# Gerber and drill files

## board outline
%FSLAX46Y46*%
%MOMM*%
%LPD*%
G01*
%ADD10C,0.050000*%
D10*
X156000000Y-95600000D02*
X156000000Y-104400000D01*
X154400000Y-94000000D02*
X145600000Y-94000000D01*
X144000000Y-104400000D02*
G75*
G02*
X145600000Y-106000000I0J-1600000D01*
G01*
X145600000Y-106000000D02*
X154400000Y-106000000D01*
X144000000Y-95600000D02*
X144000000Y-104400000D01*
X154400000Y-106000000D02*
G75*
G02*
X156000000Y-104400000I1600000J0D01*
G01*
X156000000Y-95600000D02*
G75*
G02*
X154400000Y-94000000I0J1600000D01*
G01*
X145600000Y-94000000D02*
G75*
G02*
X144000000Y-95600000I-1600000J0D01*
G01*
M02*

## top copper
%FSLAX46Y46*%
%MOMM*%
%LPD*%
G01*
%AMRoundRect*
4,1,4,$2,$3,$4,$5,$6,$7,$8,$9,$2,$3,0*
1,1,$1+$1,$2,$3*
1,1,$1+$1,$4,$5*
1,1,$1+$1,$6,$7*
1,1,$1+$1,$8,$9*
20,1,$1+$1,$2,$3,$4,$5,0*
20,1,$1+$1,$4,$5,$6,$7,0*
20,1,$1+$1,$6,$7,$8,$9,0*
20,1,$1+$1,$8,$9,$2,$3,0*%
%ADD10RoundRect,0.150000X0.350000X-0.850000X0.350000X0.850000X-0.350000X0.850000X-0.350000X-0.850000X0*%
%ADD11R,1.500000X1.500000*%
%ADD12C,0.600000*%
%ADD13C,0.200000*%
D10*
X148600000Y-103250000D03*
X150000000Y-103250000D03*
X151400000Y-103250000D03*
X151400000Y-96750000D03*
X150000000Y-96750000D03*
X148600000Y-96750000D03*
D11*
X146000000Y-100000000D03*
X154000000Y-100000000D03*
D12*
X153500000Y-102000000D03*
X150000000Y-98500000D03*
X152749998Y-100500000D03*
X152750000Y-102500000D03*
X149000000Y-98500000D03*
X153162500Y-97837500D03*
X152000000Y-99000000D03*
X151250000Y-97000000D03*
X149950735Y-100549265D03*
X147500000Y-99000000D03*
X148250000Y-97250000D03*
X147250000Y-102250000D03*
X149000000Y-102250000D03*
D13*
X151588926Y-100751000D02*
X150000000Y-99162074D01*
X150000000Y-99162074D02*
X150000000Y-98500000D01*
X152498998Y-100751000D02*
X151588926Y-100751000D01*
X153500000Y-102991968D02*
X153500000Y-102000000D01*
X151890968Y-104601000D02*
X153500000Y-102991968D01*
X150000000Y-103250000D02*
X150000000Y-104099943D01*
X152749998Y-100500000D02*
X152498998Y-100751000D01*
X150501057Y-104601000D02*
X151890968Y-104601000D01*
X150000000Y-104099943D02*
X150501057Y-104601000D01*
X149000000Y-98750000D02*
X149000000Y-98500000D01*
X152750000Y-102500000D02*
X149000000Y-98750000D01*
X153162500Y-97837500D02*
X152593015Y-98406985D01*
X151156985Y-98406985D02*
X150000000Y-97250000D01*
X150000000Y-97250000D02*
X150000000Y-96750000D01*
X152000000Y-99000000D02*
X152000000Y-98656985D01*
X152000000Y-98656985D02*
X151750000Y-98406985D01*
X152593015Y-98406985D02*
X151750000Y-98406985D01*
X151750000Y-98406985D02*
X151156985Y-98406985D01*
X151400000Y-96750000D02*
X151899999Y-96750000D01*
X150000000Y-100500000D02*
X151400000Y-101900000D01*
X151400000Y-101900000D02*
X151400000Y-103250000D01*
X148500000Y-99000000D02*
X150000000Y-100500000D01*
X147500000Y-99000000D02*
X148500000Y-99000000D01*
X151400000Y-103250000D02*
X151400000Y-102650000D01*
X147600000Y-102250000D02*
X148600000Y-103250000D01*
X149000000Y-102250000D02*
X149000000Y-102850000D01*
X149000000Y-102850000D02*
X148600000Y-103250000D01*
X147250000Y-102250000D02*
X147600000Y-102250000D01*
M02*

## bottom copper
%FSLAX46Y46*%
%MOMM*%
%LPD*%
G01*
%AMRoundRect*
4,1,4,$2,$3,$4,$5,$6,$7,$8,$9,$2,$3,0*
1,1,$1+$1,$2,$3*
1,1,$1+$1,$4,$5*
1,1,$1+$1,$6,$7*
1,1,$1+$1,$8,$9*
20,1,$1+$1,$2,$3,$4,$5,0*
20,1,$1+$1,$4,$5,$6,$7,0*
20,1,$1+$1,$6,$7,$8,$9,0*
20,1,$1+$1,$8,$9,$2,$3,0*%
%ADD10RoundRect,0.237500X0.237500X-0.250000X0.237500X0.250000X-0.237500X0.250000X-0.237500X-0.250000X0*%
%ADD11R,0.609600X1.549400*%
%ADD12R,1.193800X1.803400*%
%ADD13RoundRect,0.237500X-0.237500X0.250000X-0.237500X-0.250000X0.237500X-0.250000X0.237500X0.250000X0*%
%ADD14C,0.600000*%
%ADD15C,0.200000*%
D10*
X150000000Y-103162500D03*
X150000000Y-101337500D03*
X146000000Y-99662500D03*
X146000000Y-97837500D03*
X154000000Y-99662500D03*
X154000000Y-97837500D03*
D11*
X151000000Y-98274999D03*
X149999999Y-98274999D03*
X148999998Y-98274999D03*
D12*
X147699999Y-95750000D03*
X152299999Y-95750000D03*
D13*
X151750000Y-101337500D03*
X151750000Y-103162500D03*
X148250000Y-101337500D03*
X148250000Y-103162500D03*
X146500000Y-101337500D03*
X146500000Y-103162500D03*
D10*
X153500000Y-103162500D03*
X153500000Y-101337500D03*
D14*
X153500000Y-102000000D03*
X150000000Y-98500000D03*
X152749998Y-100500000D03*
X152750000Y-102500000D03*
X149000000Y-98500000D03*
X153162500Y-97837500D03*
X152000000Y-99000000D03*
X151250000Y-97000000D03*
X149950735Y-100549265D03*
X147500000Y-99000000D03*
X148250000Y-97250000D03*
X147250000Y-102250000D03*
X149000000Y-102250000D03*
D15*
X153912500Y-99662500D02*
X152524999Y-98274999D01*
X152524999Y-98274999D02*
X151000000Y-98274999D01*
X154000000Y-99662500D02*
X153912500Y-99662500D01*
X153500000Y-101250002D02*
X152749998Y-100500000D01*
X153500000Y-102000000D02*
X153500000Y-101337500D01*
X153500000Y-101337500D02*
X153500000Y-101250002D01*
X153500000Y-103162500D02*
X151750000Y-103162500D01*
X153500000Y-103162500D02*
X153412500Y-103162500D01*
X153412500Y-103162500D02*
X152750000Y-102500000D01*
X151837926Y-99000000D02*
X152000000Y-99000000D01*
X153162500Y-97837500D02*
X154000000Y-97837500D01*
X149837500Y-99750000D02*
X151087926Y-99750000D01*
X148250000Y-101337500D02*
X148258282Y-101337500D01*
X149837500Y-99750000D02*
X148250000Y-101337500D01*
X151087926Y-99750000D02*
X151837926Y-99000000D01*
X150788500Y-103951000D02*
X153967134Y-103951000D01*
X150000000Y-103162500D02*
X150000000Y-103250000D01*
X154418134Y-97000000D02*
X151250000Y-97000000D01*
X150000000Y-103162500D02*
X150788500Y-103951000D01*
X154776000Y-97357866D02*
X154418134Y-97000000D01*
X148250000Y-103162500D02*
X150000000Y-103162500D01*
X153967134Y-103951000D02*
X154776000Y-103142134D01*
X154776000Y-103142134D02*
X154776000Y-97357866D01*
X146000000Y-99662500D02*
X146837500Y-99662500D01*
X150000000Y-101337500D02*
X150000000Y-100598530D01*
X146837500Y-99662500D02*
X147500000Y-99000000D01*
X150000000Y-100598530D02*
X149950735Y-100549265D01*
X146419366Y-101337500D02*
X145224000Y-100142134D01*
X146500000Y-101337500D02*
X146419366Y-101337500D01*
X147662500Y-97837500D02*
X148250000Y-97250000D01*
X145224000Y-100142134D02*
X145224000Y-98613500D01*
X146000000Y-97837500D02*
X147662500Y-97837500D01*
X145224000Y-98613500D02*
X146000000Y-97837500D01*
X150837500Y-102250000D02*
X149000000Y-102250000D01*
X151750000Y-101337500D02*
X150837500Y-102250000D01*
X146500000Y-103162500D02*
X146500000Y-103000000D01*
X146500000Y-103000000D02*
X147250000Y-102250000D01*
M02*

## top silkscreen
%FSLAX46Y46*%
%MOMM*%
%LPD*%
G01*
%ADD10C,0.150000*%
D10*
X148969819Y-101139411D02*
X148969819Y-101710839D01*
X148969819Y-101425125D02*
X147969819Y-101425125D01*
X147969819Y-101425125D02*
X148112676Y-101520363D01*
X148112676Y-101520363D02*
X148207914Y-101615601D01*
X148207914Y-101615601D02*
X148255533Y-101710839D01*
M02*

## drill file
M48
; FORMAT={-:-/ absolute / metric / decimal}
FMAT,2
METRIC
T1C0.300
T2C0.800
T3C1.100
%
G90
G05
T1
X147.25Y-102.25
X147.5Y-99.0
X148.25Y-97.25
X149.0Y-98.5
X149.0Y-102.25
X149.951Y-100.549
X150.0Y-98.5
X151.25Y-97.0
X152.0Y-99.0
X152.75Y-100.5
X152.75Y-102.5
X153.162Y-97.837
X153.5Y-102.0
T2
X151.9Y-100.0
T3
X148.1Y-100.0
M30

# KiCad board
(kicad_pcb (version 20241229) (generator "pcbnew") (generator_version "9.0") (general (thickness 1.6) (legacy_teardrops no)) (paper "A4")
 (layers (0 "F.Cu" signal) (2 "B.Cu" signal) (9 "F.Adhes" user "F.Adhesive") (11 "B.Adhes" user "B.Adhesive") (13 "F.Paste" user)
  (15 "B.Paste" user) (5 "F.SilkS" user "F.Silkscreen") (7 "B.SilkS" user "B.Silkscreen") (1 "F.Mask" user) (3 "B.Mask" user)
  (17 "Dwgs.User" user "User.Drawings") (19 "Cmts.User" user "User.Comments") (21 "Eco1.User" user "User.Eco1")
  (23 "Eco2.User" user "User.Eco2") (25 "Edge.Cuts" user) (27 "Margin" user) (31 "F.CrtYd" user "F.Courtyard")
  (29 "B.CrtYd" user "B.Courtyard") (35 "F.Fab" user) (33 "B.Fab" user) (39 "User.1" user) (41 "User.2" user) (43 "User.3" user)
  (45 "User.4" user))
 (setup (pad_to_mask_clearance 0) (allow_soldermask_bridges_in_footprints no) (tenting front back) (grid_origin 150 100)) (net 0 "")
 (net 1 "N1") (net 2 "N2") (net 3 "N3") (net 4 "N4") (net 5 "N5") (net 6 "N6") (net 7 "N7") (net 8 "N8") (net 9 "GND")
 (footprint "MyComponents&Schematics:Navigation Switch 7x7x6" (layer "F.Cu") (at 150 100 90)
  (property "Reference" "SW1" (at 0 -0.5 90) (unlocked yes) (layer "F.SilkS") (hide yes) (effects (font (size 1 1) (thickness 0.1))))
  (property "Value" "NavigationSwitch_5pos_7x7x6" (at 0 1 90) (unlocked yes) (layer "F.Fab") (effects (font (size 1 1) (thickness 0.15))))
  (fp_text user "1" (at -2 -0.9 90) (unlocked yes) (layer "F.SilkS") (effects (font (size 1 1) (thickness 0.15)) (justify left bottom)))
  (pad "" np_thru_hole circle (at 0 -1.9 90) (size 1.1 1.1) (drill 1.1) (layers "*.Mask"))
  (pad "" np_thru_hole circle (at 0 1.9 90) (size 0.8 0.8) (drill 0.8) (layers "*.Mask"))
  (pad "1" smd roundrect (at -3.25 -1.4 90) (size 2 1) (layers "F.Cu" "F.Mask" "F.Paste") (roundrect_rratio 0.15) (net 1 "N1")
   (thermal_bridge_angle 45))
  (pad "2" smd roundrect (at -3.25 0 90) (size 2 1) (layers "F.Cu" "F.Mask" "F.Paste") (roundrect_rratio 0.15) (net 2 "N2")
   (thermal_bridge_angle 45))
  (pad "3" smd roundrect (at -3.25 1.4 90) (size 2 1) (layers "F.Cu" "F.Mask" "F.Paste") (roundrect_rratio 0.15) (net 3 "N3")
   (thermal_bridge_angle 45))
  (pad "4" smd roundrect (at 3.25 1.4 90) (size 2 1) (layers "F.Cu" "F.Mask" "F.Paste") (roundrect_rratio 0.15) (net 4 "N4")
   (thermal_bridge_angle 45))
  (pad "5" smd roundrect (at 3.25 0 90) (size 2 1) (layers "F.Cu" "F.Mask" "F.Paste") (roundrect_rratio 0.15) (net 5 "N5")
   (thermal_bridge_angle 45))
  (pad "6" smd roundrect (at 3.25 -1.4 90) (size 2 1) (layers "F.Cu" "F.Mask" "F.Paste") (roundrect_rratio 0.15) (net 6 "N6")
   (thermal_bridge_angle 45))
  (pad "MP" smd rect (at 0 -4 90) (size 1.5 1.5) (layers "F.Cu" "F.Mask" "F.Paste") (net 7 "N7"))
  (pad "MP" smd rect (at 0 4 90) (size 1.5 1.5) (layers "F.Cu" "F.Mask" "F.Paste") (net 7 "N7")))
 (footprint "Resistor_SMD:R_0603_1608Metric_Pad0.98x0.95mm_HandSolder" (layer "B.Cu") (at 150 102.25 90)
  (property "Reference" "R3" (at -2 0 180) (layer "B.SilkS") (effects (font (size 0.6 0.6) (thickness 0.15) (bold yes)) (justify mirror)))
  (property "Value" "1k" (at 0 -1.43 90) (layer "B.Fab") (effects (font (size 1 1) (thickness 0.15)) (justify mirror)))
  (pad "1" smd roundrect (at -0.9125 0 90) (size 0.975 0.95) (layers "B.Cu" "B.Mask" "B.Paste") (roundrect_rratio 0.25) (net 4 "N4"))
  (pad "2" smd roundrect (at 0.9125 0 90) (size 0.975 0.95) (layers "B.Cu" "B.Mask" "B.Paste") (roundrect_rratio 0.25) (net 3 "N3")))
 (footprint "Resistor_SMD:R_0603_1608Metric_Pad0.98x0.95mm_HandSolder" (layer "B.Cu") (at 146 98.75 90)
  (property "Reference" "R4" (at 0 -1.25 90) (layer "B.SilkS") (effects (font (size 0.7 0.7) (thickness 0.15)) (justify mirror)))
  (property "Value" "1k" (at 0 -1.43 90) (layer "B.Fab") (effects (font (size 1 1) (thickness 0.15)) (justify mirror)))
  (pad "1" smd roundrect (at -0.9125 0 90) (size 0.975 0.95) (layers "B.Cu" "B.Mask" "B.Paste") (roundrect_rratio 0.25) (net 3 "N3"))
  (pad "2" smd roundrect (at 0.9125 0 90) (size 0.975 0.95) (layers "B.Cu" "B.Mask" "B.Paste") (roundrect_rratio 0.25) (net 6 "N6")))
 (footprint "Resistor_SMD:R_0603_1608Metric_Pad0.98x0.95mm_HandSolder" (layer "B.Cu") (at 154 98.75 90)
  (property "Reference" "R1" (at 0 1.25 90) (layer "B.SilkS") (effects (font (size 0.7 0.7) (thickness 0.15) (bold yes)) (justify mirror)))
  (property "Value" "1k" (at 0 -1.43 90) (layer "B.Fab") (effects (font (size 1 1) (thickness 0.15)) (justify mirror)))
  (pad "1" smd roundrect (at -0.9125 0 90) (size 0.975 0.95) (layers "B.Cu" "B.Mask" "B.Paste") (roundrect_rratio 0.25) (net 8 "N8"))
  (pad "2" smd roundrect (at 0.9125 0 90) (size 0.975 0.95) (layers "B.Cu" "B.Mask" "B.Paste") (roundrect_rratio 0.25) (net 5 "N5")))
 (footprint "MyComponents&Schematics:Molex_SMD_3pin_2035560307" (layer "B.Cu") (at 149.999999 96.551399)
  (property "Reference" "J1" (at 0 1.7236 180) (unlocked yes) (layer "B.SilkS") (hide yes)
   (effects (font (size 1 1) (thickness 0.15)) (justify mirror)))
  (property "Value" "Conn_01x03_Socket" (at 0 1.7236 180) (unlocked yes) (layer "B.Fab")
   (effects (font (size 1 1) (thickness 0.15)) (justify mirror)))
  (pad "1" smd rect (at 1.000001 1.7236) (size 0.6096 1.5494) (layers "B.Cu" "B.Mask" "B.Paste") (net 8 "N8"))
  (pad "2" smd rect (at 0 1.7236) (size 0.6096 1.5494) (layers "B.Cu" "B.Mask" "B.Paste") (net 2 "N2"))
  (pad "3" smd rect (at -1.000001 1.7236) (size 0.6096 1.5494) (layers "B.Cu" "B.Mask" "B.Paste") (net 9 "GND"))
  (pad "4" smd rect (at -2.3 -0.801399) (size 1.1938 1.8034) (layers "B.Cu" "B.Mask" "B.Paste"))
  (pad "5" smd rect (at 2.3 -0.801399) (size 1.1938 1.8034) (layers "B.Cu" "B.Mask" "B.Paste")))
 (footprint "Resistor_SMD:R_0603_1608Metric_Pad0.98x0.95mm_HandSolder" (layer "B.Cu") (at 151.75 102.25 -90)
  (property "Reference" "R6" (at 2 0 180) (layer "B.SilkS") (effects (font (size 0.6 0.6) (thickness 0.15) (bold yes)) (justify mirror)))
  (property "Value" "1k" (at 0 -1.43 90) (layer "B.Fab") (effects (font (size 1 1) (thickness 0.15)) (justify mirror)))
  (pad "1" smd roundrect (at -0.9125 0 270) (size 0.975 0.95) (layers "B.Cu" "B.Mask" "B.Paste") (roundrect_rratio 0.25) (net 1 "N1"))
  (pad "2" smd roundrect (at 0.9125 0 270) (size 0.975 0.95) (layers "B.Cu" "B.Mask" "B.Paste") (roundrect_rratio 0.25) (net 9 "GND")))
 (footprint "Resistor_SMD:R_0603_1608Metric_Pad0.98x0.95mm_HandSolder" (layer "B.Cu") (at 148.25 102.25 -90)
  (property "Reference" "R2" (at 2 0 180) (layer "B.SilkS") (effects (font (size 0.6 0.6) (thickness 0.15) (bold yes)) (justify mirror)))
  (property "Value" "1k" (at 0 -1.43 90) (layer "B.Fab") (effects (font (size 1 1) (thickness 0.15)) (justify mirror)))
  (pad "1" smd roundrect (at -0.9125 0 270) (size 0.975 0.95) (layers "B.Cu" "B.Mask" "B.Paste") (roundrect_rratio 0.25) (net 5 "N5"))
  (pad "2" smd roundrect (at 0.9125 0 270) (size 0.975 0.95) (layers "B.Cu" "B.Mask" "B.Paste") (roundrect_rratio 0.25) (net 4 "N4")))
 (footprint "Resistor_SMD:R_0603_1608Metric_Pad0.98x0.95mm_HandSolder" (layer "B.Cu") (at 146.5 102.25 -90)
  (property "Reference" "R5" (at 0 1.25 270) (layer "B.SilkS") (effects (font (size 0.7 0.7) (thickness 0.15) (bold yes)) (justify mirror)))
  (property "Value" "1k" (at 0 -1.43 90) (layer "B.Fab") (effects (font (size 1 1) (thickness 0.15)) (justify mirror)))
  (pad "1" smd roundrect (at -0.9125 0 270) (size 0.975 0.95) (layers "B.Cu" "B.Mask" "B.Paste") (roundrect_rratio 0.25) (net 6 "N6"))
  (pad "2" smd roundrect (at 0.9125 0 270) (size 0.975 0.95) (layers "B.Cu" "B.Mask" "B.Paste") (roundrect_rratio 0.25) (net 1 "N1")))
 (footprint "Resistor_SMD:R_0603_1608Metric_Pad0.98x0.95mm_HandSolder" (layer "B.Cu") (at 153.5 102.25 90)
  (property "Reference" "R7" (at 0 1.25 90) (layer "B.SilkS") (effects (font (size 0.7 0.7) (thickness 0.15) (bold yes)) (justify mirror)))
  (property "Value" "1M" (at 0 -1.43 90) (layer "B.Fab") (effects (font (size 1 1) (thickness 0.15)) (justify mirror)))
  (pad "1" smd roundrect (at -0.9125 0 90) (size 0.975 0.95) (layers "B.Cu" "B.Mask" "B.Paste") (roundrect_rratio 0.25) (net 9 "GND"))
  (pad "2" smd roundrect (at 0.9125 0 90) (size 0.975 0.95) (layers "B.Cu" "B.Mask" "B.Paste") (roundrect_rratio 0.25) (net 2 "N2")))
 (gr_line (start 156 95.6) (end 156 104.4) (stroke (width 0.05) (type default)) (layer "Edge.Cuts"))
 (gr_line (start 154.4 94) (end 145.6 94) (stroke (width 0.05) (type default)) (layer "Edge.Cuts"))
 (gr_arc (start 144 104.4) (mid 145.131371 104.868629) (end 145.6 106) (stroke (width 0.05) (type default)) (layer "Edge.Cuts"))
 (gr_line (start 145.6 106) (end 154.4 106) (stroke (width 0.05) (type default)) (layer "Edge.Cuts"))
 (gr_line (start 144 95.6) (end 144 104.4) (stroke (width 0.05) (type default)) (layer "Edge.Cuts"))
 (gr_arc (start 154.4 106) (mid 154.868629 104.868629) (end 156 104.4) (stroke (width 0.05) (type default)) (layer "Edge.Cuts"))
 (gr_arc (start 156 95.6) (mid 154.868629 95.131371) (end 154.4 94) (stroke (width 0.05) (type default)) (layer "Edge.Cuts"))
 (gr_arc (start 145.6 94) (mid 145.131371 95.131371) (end 144 95.6) (stroke (width 0.05) (type default)) (layer "Edge.Cuts"))
 (segment (start 153.9125 99.6625) (end 152.524999 98.274999) (width 0.2) (layer "B.Cu") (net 8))
 (segment (start 152.524999 98.274999) (end 151 98.274999) (width 0.2) (layer "B.Cu") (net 8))
 (segment (start 154 99.6625) (end 153.9125 99.6625) (width 0.2) (layer "B.Cu") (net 8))
 (segment (start 151.588926 100.751) (end 150 99.162074) (width 0.2) (layer "F.Cu") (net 2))
 (segment (start 150 99.162074) (end 150 98.5) (width 0.2) (layer "F.Cu") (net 2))
 (segment (start 152.498998 100.751) (end 151.588926 100.751) (width 0.2) (layer "F.Cu") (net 2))
 (segment (start 153.5 102.991968) (end 153.5 102) (width 0.2) (layer "F.Cu") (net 2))
 (segment (start 151.890968 104.601) (end 153.5 102.991968) (width 0.2) (layer "F.Cu") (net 2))
 (segment (start 150 103.25) (end 150 104.099943) (width 0.2) (layer "F.Cu") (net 2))
 (segment (start 152.749998 100.5) (end 152.498998 100.751) (width 0.2) (layer "F.Cu") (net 2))
 (segment (start 150.501057 104.601) (end 151.890968 104.601) (width 0.2) (layer "F.Cu") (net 2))
 (segment (start 150 104.099943) (end 150.501057 104.601) (width 0.2) (layer "F.Cu") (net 2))
 (via (at 153.5 102) (size 0.6) (drill 0.3) (layers "F.Cu" "B.Cu") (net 2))
 (via (at 150 98.5) (size 0.6) (drill 0.3) (layers "F.Cu" "B.Cu") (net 2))
 (via (at 152.749998 100.5) (size 0.6) (drill 0.3) (layers "F.Cu" "B.Cu") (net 2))
 (segment (start 153.5 101.250002) (end 152.749998 100.5) (width 0.2) (layer "B.Cu") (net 2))
 (segment (start 153.5 102) (end 153.5 101.3375) (width 0.2) (layer "B.Cu") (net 2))
 (segment (start 153.5 101.3375) (end 153.5 101.250002) (width 0.2) (layer "B.Cu") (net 2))
 (segment (start 149 98.75) (end 149 98.5) (width 0.2) (layer "F.Cu") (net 9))
 (segment (start 152.75 102.5) (end 149 98.75) (width 0.2) (layer "F.Cu") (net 9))
 (via (at 152.75 102.5) (size 0.6) (drill 0.3) (layers "F.Cu" "B.Cu") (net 9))
 (via (at 149 98.5) (size 0.6) (drill 0.3) (layers "F.Cu" "B.Cu") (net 9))
 (segment (start 153.5 103.1625) (end 151.75 103.1625) (width 0.2) (layer "B.Cu") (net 9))
 (segment (start 153.5 103.1625) (end 153.4125 103.1625) (width 0.2) (layer "B.Cu") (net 9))
 (segment (start 153.4125 103.1625) (end 152.75 102.5) (width 0.2) (layer "B.Cu") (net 9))
 (segment (start 153.1625 97.8375) (end 152.593015 98.406985) (width 0.2) (layer "F.Cu") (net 5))
 (segment (start 151.156985 98.406985) (end 150 97.25) (width 0.2) (layer "F.Cu") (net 5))
 (segment (start 150 97.25) (end 150 96.75) (width 0.2) (layer "F.Cu") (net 5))
 (segment (start 152 99) (end 152 98.656985) (width 0.2) (layer "F.Cu") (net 5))
 (segment (start 152 98.656985) (end 151.75 98.406985) (width 0.2) (layer "F.Cu") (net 5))
 (segment (start 152.593015 98.406985) (end 151.75 98.406985) (width 0.2) (layer "F.Cu") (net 5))
 (segment (start 151.75 98.406985) (end 151.156985 98.406985) (width 0.2) (layer "F.Cu") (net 5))
 (via (at 153.1625 97.8375) (size 0.6) (drill 0.3) (layers "F.Cu" "B.Cu") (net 5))
 (via (at 152 99) (size 0.6) (drill 0.3) (layers "F.Cu" "B.Cu") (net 5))
 (segment (start 151.837926 99) (end 152 99) (width 0.2) (layer "B.Cu") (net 5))
 (segment (start 153.1625 97.8375) (end 154 97.8375) (width 0.2) (layer "B.Cu") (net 5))
 (segment (start 149.8375 99.75) (end 151.087926 99.75) (width 0.2) (layer "B.Cu") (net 5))
 (segment (start 148.25 101.3375) (end 148.258282 101.3375) (width 0.2) (layer "B.Cu") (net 5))
 (segment (start 149.8375 99.75) (end 148.25 101.3375) (width 0.2) (layer "B.Cu") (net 5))
 (segment (start 151.087926 99.75) (end 151.837926 99) (width 0.2) (layer "B.Cu") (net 5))
 (segment (start 151.4 96.75) (end 151.899999 96.75) (width 0.2) (layer "F.Cu") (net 4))
 (via (at 151.25 97) (size 0.6) (drill 0.3) (layers "F.Cu" "B.Cu") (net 4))
 (segment (start 150.7885 103.951) (end 153.967134 103.951) (width 0.2) (layer "B.Cu") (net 4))
 (segment (start 150 103.1625) (end 150 103.25) (width 0.2) (layer "B.Cu") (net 4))
 (segment (start 154.418134 97) (end 151.25 97) (width 0.2) (layer "B.Cu") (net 4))
 (segment (start 150 103.1625) (end 150.7885 103.951) (width 0.2) (layer "B.Cu") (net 4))
 (segment (start 154.776 97.357866) (end 154.418134 97) (width 0.2) (layer "B.Cu") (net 4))
 (segment (start 148.25 103.1625) (end 150 103.1625) (width 0.2) (layer "B.Cu") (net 4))
 (segment (start 153.967134 103.951) (end 154.776 103.142134) (width 0.2) (layer "B.Cu") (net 4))
 (segment (start 154.776 103.142134) (end 154.776 97.357866) (width 0.2) (layer "B.Cu") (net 4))
 (segment (start 150 100.5) (end 151.4 101.9) (width 0.2) (layer "F.Cu") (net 3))
 (segment (start 151.4 101.9) (end 151.4 103.25) (width 0.2) (layer "F.Cu") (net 3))
 (segment (start 148.5 99) (end 150 100.5) (width 0.2) (layer "F.Cu") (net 3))
 (segment (start 147.5 99) (end 148.5 99) (width 0.2) (layer "F.Cu") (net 3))
 (segment (start 151.4 103.25) (end 151.4 102.65) (width 0.2) (layer "F.Cu") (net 3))
 (via (at 149.950735 100.549265) (size 0.6) (drill 0.3) (layers "F.Cu" "B.Cu") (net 3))
 (via (at 147.5 99) (size 0.6) (drill 0.3) (layers "F.Cu" "B.Cu") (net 3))
 (segment (start 146 99.6625) (end 146.8375 99.6625) (width 0.2) (layer "B.Cu") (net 3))
 (segment (start 150 101.3375) (end 150 100.59853) (width 0.2) (layer "B.Cu") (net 3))
 (segment (start 146.8375 99.6625) (end 147.5 99) (width 0.2) (layer "B.Cu") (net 3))
 (segment (start 150 100.59853) (end 149.950735 100.549265) (width 0.2) (layer "B.Cu") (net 3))
 (via (at 148.25 97.25) (size 0.6) (drill 0.3) (layers "F.Cu" "B.Cu") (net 6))
 (segment (start 146.419366 101.3375) (end 145.224 100.142134) (width 0.2) (layer "B.Cu") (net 6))
 (segment (start 146.5 101.3375) (end 146.419366 101.3375) (width 0.2) (layer "B.Cu") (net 6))
 (segment (start 147.6625 97.8375) (end 148.25 97.25) (width 0.2) (layer "B.Cu") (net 6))
 (segment (start 145.224 100.142134) (end 145.224 98.6135) (width 0.2) (layer "B.Cu") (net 6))
 (segment (start 146 97.8375) (end 147.6625 97.8375) (width 0.2) (layer "B.Cu") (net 6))
 (segment (start 145.224 98.6135) (end 146 97.8375) (width 0.2) (layer "B.Cu") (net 6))
 (segment (start 147.6 102.25) (end 148.6 103.25) (width 0.2) (layer "F.Cu") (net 1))
 (segment (start 149 102.25) (end 149 102.85) (width 0.2) (layer "F.Cu") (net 1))
 (segment (start 149 102.85) (end 148.6 103.25) (width 0.2) (layer "F.Cu") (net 1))
 (segment (start 147.25 102.25) (end 147.6 102.25) (width 0.2) (layer "F.Cu") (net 1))
 (via (at 147.25 102.25) (size 0.6) (drill 0.3) (layers "F.Cu" "B.Cu") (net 1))
 (via (at 149 102.25) (size 0.6) (drill 0.3) (layers "F.Cu" "B.Cu") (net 1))
 (segment (start 150.8375 102.25) (end 149 102.25) (width 0.2) (layer "B.Cu") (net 1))
 (segment (start 151.75 101.3375) (end 150.8375 102.25) (width 0.2) (layer "B.Cu") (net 1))
 (segment (start 146.5 103.1625) (end 146.5 103) (width 0.2) (layer "B.Cu") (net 1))
 (segment (start 146.5 103) (end 147.25 102.25) (width 0.2) (layer "B.Cu") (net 1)))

